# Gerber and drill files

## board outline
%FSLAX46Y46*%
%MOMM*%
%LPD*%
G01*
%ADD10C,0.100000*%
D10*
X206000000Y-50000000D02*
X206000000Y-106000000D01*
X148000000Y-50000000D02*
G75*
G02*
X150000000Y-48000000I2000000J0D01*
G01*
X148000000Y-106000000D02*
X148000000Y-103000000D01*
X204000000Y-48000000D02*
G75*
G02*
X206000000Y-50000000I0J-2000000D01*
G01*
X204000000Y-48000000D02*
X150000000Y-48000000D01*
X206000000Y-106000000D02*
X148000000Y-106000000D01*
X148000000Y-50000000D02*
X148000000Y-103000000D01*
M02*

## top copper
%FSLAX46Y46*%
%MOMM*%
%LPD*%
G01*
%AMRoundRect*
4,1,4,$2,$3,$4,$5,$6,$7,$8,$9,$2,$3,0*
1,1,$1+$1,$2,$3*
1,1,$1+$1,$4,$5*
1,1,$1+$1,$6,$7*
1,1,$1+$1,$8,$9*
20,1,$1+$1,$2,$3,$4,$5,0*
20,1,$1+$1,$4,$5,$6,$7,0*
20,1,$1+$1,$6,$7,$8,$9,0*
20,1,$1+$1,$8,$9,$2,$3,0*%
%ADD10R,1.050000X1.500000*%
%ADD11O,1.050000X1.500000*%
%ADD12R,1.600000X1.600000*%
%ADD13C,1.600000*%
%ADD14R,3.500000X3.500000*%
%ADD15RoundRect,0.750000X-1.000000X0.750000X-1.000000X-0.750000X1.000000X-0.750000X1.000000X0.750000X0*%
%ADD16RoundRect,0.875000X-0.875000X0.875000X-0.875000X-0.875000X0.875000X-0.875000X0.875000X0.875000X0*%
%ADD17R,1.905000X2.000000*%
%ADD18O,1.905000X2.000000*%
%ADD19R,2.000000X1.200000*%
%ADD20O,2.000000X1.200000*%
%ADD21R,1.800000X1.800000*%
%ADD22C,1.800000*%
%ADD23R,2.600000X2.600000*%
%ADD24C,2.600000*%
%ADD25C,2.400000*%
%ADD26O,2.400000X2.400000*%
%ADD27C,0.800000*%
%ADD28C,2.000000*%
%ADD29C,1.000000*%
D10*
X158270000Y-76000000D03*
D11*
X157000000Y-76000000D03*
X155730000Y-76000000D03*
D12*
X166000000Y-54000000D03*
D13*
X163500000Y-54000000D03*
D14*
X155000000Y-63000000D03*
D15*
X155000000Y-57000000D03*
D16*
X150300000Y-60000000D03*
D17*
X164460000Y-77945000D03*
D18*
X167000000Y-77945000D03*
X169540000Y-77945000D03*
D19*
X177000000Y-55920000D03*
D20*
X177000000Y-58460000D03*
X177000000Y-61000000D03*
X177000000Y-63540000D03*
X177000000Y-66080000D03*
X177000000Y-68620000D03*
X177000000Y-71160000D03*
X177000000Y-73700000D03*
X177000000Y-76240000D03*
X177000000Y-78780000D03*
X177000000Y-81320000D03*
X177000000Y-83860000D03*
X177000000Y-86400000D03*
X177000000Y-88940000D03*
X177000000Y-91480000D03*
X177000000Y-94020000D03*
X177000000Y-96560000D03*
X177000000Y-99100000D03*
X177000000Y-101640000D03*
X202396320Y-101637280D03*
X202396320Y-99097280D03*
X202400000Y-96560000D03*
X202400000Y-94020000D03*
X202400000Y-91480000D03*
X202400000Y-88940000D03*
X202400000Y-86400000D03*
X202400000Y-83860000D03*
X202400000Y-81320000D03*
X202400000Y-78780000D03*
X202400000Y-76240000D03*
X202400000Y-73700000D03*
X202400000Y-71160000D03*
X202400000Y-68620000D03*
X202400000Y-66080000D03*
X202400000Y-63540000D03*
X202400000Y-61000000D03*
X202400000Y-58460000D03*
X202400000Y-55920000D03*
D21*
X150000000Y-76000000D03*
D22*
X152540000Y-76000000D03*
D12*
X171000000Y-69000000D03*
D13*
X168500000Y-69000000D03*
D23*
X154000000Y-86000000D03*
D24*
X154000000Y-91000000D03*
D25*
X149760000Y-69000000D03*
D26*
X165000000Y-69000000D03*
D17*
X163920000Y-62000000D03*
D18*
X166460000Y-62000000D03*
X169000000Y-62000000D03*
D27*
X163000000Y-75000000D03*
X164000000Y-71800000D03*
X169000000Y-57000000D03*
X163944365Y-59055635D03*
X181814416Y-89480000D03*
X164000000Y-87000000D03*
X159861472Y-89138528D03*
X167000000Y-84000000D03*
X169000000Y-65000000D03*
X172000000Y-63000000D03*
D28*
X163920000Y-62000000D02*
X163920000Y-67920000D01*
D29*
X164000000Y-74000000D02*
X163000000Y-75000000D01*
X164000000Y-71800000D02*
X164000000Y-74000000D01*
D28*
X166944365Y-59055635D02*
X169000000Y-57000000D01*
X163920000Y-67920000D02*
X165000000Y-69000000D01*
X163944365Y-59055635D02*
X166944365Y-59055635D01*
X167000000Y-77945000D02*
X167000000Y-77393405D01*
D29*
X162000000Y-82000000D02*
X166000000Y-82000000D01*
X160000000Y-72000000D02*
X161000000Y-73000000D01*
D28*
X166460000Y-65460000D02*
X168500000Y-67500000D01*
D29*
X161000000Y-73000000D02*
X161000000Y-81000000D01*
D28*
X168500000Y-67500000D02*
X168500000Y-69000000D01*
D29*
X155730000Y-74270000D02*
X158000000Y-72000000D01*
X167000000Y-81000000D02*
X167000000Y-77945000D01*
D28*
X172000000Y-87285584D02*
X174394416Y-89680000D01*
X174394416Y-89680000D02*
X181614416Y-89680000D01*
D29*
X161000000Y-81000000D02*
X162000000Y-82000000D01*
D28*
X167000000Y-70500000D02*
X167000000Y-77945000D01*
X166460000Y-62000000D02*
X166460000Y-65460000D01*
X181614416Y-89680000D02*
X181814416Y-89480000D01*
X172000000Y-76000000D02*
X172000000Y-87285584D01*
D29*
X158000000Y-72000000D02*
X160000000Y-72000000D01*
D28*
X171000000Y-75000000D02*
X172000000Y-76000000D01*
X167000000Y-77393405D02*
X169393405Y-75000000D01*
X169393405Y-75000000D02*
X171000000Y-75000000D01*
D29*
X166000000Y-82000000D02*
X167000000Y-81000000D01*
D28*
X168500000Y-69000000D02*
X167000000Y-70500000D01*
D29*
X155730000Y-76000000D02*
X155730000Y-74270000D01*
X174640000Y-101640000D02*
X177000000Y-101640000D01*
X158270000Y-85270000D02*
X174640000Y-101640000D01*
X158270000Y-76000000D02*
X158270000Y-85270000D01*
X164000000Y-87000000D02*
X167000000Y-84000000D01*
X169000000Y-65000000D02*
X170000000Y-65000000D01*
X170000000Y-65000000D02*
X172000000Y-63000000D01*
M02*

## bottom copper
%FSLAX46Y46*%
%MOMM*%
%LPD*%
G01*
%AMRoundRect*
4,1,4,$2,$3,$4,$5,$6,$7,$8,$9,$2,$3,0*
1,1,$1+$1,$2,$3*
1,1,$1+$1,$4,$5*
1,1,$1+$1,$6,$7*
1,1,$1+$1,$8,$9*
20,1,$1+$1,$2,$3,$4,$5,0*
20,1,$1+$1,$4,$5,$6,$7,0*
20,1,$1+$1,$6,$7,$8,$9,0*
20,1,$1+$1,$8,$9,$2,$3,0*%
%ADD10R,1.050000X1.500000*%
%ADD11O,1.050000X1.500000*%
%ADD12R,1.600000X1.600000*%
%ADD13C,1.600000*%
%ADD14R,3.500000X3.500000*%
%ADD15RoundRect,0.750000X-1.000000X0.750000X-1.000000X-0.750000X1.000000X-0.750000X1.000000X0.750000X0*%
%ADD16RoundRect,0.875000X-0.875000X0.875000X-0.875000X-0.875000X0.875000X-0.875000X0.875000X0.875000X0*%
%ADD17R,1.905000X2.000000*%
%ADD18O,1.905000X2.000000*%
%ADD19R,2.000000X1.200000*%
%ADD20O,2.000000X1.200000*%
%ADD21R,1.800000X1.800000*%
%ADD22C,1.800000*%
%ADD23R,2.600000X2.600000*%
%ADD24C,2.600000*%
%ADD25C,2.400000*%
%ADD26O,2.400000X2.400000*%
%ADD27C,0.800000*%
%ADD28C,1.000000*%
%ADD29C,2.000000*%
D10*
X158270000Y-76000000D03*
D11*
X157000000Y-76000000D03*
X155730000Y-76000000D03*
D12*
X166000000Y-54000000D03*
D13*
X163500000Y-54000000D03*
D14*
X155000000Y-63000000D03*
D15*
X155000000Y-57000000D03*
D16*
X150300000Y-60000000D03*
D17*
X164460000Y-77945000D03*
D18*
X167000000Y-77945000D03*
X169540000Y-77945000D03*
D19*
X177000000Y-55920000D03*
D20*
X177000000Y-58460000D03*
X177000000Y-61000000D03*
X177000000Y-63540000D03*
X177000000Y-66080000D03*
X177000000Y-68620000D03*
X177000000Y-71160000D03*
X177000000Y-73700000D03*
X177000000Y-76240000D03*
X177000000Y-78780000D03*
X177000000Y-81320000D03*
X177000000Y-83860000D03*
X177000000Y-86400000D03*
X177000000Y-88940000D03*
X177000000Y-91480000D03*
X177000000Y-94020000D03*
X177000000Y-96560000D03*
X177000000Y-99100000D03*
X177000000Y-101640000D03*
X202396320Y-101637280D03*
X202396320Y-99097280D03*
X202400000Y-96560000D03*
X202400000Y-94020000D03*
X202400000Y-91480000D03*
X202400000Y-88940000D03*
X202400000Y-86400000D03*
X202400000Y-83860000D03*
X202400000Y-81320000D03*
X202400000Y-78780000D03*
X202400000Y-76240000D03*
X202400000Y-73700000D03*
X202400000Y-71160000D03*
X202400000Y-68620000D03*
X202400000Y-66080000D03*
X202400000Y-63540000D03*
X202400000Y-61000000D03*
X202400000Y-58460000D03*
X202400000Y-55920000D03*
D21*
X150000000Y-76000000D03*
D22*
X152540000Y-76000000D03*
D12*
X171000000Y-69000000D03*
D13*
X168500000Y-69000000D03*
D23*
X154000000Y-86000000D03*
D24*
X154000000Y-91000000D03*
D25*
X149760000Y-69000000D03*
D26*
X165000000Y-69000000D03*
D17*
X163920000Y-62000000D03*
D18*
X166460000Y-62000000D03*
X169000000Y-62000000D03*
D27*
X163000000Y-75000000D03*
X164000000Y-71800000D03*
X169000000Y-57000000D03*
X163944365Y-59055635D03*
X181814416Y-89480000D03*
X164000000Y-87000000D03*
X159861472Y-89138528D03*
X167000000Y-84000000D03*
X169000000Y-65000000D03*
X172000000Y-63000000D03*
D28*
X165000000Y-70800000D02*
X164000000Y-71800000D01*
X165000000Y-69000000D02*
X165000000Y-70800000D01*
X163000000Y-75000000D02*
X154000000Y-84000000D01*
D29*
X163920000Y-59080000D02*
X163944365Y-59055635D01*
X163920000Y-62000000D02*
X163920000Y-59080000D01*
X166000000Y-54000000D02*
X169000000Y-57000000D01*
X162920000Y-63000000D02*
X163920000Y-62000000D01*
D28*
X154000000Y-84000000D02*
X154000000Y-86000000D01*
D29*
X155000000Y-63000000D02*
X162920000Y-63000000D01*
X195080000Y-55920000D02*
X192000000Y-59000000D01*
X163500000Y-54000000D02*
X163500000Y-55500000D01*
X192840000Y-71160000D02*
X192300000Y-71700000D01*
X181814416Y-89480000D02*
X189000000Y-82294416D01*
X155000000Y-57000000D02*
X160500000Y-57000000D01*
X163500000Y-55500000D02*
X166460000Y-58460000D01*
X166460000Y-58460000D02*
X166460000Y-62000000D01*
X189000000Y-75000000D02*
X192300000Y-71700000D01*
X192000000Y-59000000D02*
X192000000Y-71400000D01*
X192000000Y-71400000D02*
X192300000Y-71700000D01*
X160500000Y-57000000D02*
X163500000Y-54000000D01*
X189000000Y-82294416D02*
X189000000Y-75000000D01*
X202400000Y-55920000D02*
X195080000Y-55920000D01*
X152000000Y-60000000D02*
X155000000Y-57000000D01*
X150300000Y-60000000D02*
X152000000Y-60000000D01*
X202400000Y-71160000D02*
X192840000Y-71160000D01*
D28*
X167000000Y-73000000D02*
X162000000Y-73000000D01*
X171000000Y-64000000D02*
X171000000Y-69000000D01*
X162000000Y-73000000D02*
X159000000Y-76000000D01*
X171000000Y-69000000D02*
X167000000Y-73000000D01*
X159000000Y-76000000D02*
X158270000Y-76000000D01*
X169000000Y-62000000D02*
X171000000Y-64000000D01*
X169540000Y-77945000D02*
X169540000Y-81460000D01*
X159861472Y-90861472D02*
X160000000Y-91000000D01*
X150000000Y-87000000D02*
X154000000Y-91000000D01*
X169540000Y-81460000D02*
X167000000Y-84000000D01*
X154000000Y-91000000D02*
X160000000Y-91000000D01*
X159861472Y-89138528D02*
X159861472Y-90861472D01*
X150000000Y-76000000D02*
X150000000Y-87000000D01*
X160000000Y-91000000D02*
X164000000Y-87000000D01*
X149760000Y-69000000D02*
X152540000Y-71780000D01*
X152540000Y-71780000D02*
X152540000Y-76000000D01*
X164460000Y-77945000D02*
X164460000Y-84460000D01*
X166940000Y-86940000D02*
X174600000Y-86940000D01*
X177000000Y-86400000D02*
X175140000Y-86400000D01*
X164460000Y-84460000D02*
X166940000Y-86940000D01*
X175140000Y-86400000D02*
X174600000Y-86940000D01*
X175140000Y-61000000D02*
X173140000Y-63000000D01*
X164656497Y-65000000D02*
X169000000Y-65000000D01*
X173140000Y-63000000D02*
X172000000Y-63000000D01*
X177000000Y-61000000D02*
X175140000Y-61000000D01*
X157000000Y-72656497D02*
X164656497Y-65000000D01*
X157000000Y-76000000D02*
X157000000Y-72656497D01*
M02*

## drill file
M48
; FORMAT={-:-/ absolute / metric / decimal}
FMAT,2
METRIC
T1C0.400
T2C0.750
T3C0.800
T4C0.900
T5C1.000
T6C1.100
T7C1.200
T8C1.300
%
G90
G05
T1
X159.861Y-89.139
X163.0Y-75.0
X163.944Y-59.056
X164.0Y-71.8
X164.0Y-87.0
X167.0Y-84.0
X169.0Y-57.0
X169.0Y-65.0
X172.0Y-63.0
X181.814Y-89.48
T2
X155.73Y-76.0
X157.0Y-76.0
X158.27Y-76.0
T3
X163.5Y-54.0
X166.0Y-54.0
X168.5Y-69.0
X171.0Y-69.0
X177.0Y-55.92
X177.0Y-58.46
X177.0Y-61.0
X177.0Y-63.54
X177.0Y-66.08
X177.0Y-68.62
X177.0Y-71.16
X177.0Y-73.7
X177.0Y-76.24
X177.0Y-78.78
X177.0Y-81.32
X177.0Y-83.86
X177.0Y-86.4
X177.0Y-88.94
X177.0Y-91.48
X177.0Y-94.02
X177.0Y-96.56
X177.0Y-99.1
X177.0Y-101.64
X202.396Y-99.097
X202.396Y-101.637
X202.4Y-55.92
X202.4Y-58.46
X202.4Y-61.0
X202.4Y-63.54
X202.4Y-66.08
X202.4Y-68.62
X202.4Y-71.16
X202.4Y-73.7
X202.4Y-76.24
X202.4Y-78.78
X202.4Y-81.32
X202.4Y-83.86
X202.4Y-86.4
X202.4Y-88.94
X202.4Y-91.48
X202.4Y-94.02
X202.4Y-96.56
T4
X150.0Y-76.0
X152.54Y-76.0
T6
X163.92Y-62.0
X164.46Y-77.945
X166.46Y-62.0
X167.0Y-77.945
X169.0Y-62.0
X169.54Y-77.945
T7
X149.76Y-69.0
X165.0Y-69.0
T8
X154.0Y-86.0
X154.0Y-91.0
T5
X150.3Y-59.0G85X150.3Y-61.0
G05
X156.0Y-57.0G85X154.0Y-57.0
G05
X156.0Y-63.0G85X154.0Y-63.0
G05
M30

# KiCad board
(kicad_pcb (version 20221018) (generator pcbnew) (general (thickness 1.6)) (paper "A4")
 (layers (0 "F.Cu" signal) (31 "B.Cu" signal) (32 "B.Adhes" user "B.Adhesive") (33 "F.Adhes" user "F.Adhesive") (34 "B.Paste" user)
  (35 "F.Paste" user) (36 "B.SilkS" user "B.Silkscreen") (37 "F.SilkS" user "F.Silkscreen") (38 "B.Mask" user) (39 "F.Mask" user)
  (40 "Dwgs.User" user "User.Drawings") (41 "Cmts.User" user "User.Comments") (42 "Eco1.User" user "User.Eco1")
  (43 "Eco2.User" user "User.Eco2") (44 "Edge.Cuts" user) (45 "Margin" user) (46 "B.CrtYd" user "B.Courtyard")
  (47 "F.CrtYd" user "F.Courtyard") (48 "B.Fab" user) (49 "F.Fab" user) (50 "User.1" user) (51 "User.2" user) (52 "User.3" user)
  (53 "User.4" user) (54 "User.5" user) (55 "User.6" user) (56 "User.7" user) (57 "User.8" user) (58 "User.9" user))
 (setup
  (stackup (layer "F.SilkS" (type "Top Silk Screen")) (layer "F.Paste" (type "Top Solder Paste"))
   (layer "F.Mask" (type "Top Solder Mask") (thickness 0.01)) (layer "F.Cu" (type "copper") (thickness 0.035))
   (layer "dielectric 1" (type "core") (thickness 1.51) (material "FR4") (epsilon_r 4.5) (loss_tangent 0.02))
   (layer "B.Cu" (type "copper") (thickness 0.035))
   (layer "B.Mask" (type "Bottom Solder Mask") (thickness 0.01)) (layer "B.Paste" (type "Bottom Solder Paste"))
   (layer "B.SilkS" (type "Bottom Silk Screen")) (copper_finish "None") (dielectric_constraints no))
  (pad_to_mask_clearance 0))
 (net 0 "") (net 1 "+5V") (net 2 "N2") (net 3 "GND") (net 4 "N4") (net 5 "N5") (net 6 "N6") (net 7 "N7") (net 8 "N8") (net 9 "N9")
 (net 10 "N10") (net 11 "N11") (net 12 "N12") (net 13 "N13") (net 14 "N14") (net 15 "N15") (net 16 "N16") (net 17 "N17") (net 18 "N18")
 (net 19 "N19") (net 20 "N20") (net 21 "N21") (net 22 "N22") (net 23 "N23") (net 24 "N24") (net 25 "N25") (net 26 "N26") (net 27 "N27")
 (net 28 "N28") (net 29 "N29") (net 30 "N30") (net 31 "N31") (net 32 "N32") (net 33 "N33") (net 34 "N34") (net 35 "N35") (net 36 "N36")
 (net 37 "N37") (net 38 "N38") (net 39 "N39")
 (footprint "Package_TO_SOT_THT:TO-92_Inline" (layer "F.Cu") (at 158.27 76 180)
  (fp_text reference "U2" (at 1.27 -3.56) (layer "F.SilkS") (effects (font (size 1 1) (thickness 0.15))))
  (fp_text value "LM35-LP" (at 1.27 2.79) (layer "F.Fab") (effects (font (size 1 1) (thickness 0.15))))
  (pad "1" thru_hole rect (at 0 0 180) (size 1.05 1.5) (drill 0.75) (layers "*.Cu" "*.Mask") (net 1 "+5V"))
  (pad "2" thru_hole oval (at 1.27 0 180) (size 1.05 1.5) (drill 0.75) (layers "*.Cu" "*.Mask") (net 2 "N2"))
  (pad "3" thru_hole oval (at 2.54 0 180) (size 1.05 1.5) (drill 0.75) (layers "*.Cu" "*.Mask") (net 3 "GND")))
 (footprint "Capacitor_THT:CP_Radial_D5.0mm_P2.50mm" (layer "F.Cu") (at 166 54 180)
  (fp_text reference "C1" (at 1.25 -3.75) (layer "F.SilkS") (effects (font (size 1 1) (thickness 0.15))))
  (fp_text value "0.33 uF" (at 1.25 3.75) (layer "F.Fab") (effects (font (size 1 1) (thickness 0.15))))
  (pad "1" thru_hole rect (at 0 0 180) (size 1.6 1.6) (drill 0.8) (layers "*.Cu" "*.Mask") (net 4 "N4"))
  (pad "2" thru_hole circle (at 2.5 0 180) (size 1.6 1.6) (drill 0.8) (layers "*.Cu" "*.Mask") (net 3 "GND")))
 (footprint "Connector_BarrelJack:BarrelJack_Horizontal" (layer "F.Cu") (at 155 63 -90)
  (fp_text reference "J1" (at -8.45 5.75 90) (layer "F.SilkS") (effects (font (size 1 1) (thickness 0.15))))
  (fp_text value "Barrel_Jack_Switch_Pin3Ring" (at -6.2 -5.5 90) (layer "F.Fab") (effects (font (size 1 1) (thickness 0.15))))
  (pad "1" thru_hole rect (at 0 0 270) (size 3.5 3.5) (drill oval 1 3) (layers "*.Cu" "*.Mask") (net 4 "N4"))
  (pad "2" thru_hole roundrect (at -6 0 270) (size 3 3.5) (drill oval 1 3) (layers "*.Cu" "*.Mask") (roundrect_rratio 0.25) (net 3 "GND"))
  (pad "3" thru_hole roundrect (at -3 4.7 270) (size 3.5 3.5) (drill oval 3 1) (layers "*.Cu" "*.Mask") (roundrect_rratio 0.25)
   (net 3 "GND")))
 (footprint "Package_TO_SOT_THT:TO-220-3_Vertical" (layer "F.Cu") (at 164.46 77.945)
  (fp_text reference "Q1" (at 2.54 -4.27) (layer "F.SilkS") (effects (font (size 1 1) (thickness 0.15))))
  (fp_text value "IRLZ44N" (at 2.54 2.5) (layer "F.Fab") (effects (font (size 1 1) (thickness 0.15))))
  (pad "1" thru_hole rect (at 0 0) (size 1.905 2) (drill 1.1) (layers "*.Cu" "*.Mask") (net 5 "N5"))
  (pad "2" thru_hole oval (at 2.54 0) (size 1.905 2) (drill 1.1) (layers "*.Cu" "*.Mask") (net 3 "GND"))
  (pad "3" thru_hole oval (at 5.08 0) (size 1.905 2) (drill 1.1) (layers "*.Cu" "*.Mask") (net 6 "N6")))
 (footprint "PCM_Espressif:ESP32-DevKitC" (layer "F.Cu") (at 177 55.92)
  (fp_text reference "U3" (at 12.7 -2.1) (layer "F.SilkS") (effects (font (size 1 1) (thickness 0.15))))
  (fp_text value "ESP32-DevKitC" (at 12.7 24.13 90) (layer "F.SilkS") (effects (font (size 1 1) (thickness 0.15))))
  (pad "1" thru_hole rect (at 0 0 270) (size 1.2 2) (drill 0.8) (layers "*.Cu" "*.Mask") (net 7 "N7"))
  (pad "2" thru_hole oval (at 0 2.54 270) (size 1.2 2) (drill 0.8) (layers "*.Cu" "*.Mask") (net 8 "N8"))
  (pad "3" thru_hole oval (at 0 5.08 270) (size 1.2 2) (drill 0.8) (layers "*.Cu" "*.Mask") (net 2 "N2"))
  (pad "4" thru_hole oval (at 0 7.62 270) (size 1.2 2) (drill 0.8) (layers "*.Cu" "*.Mask") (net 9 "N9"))
  (pad "5" thru_hole oval (at 0 10.16 270) (size 1.2 2) (drill 0.8) (layers "*.Cu" "*.Mask") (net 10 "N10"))
  (pad "6" thru_hole oval (at 0 12.7 270) (size 1.2 2) (drill 0.8) (layers "*.Cu" "*.Mask") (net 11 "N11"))
  (pad "7" thru_hole oval (at 0 15.24 270) (size 1.2 2) (drill 0.8) (layers "*.Cu" "*.Mask") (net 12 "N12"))
  (pad "8" thru_hole oval (at 0 17.78 270) (size 1.2 2) (drill 0.8) (layers "*.Cu" "*.Mask") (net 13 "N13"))
  (pad "9" thru_hole oval (at 0 20.32 270) (size 1.2 2) (drill 0.8) (layers "*.Cu" "*.Mask") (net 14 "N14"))
  (pad "10" thru_hole oval (at 0 22.86 270) (size 1.2 2) (drill 0.8) (layers "*.Cu" "*.Mask") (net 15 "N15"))
  (pad "11" thru_hole oval (at 0 25.4 270) (size 1.2 2) (drill 0.8) (layers "*.Cu" "*.Mask") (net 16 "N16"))
  (pad "12" thru_hole oval (at 0 27.94 270) (size 1.2 2) (drill 0.8) (layers "*.Cu" "*.Mask") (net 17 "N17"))
  (pad "13" thru_hole oval (at 0 30.48 270) (size 1.2 2) (drill 0.8) (layers "*.Cu" "*.Mask") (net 5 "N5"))
  (pad "14" thru_hole oval (at 0 33.02 270) (size 1.2 2) (drill 0.8) (layers "*.Cu" "*.Mask") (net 3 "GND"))
  (pad "15" thru_hole oval (at 0 35.56 270) (size 1.2 2) (drill 0.8) (layers "*.Cu" "*.Mask") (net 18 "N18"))
  (pad "16" thru_hole oval (at 0 38.1 270) (size 1.2 2) (drill 0.8) (layers "*.Cu" "*.Mask") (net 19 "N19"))
  (pad "17" thru_hole oval (at 0 40.64 270) (size 1.2 2) (drill 0.8) (layers "*.Cu" "*.Mask") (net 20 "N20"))
  (pad "18" thru_hole oval (at 0 43.18 270) (size 1.2 2) (drill 0.8) (layers "*.Cu" "*.Mask") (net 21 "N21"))
  (pad "19" thru_hole oval (at 0 45.72 270) (size 1.2 2) (drill 0.8) (layers "*.Cu" "*.Mask") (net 1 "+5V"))
  (pad "20" thru_hole oval (at 25.39632 45.71728 270) (size 1.2 2) (drill 0.8) (layers "*.Cu" "*.Mask") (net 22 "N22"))
  (pad "21" thru_hole oval (at 25.39632 43.17728 270) (size 1.2 2) (drill 0.8) (layers "*.Cu" "*.Mask") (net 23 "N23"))
  (pad "22" thru_hole oval (at 25.4 40.64 270) (size 1.2 2) (drill 0.8) (layers "*.Cu" "*.Mask") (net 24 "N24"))
  (pad "23" thru_hole oval (at 25.4 38.1 270) (size 1.2 2) (drill 0.8) (layers "*.Cu" "*.Mask") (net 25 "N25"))
  (pad "24" thru_hole oval (at 25.4 35.56 270) (size 1.2 2) (drill 0.8) (layers "*.Cu" "*.Mask") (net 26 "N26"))
  (pad "25" thru_hole oval (at 25.4 33.02 270) (size 1.2 2) (drill 0.8) (layers "*.Cu" "*.Mask") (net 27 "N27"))
  (pad "26" thru_hole oval (at 25.4 30.48 270) (size 1.2 2) (drill 0.8) (layers "*.Cu" "*.Mask") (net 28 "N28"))
  (pad "27" thru_hole oval (at 25.4 27.94 270) (size 1.2 2) (drill 0.8) (layers "*.Cu" "*.Mask") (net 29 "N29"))
  (pad "28" thru_hole oval (at 25.4 25.4 270) (size 1.2 2) (drill 0.8) (layers "*.Cu" "*.Mask") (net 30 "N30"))
  (pad "29" thru_hole oval (at 25.4 22.86 270) (size 1.2 2) (drill 0.8) (layers "*.Cu" "*.Mask") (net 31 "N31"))
  (pad "30" thru_hole oval (at 25.4 20.32 270) (size 1.2 2) (drill 0.8) (layers "*.Cu" "*.Mask") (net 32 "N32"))
  (pad "31" thru_hole oval (at 25.4 17.78 270) (size 1.2 2) (drill 0.8) (layers "*.Cu" "*.Mask") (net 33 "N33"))
  (pad "32" thru_hole oval (at 25.4 15.24 270) (size 1.2 2) (drill 0.8) (layers "*.Cu" "*.Mask") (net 3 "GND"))
  (pad "33" thru_hole oval (at 25.4 12.7 270) (size 1.2 2) (drill 0.8) (layers "*.Cu" "*.Mask") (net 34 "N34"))
  (pad "34" thru_hole oval (at 25.4 10.16 270) (size 1.2 2) (drill 0.8) (layers "*.Cu" "*.Mask") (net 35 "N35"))
  (pad "35" thru_hole oval (at 25.4 7.62 270) (size 1.2 2) (drill 0.8) (layers "*.Cu" "*.Mask") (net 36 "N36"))
  (pad "36" thru_hole oval (at 25.4 5.08 270) (size 1.2 2) (drill 0.8) (layers "*.Cu" "*.Mask") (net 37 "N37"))
  (pad "37" thru_hole oval (at 25.4 2.54 270) (size 1.2 2) (drill 0.8) (layers "*.Cu" "*.Mask") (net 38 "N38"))
  (pad "38" thru_hole oval (at 25.4 0 270) (size 1.2 2) (drill 0.8) (layers "*.Cu" "*.Mask") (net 3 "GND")))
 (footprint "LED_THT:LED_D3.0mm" (layer "F.Cu") (at 150 76)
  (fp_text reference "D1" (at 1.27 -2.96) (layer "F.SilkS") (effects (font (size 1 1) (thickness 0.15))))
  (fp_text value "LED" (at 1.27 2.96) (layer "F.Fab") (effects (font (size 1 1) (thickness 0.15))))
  (pad "1" thru_hole rect (at 0 0) (size 1.8 1.8) (drill 0.9) (layers "*.Cu" "*.Mask") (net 6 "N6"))
  (pad "2" thru_hole circle (at 2.54 0) (size 1.8 1.8) (drill 0.9) (layers "*.Cu" "*.Mask") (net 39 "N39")))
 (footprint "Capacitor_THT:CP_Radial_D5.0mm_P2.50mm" (layer "F.Cu") (at 171 69 180)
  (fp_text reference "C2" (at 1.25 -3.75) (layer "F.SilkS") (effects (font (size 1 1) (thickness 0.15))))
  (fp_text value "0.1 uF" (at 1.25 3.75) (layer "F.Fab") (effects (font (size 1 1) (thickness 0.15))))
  (pad "1" thru_hole rect (at 0 0 180) (size 1.6 1.6) (drill 0.8) (layers "*.Cu" "*.Mask") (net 1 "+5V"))
  (pad "2" thru_hole circle (at 2.5 0 180) (size 1.6 1.6) (drill 0.8) (layers "*.Cu" "*.Mask") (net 3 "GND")))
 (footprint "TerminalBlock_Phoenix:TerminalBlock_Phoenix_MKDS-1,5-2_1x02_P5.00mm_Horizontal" (layer "F.Cu") (at 154 86 -90)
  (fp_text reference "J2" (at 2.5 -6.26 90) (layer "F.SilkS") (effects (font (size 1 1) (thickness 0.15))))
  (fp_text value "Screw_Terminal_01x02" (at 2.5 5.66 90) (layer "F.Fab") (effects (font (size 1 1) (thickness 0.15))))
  (pad "1" thru_hole rect (at 0 0 270) (size 2.6 2.6) (drill 1.3) (layers "*.Cu" "*.Mask") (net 4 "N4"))
  (pad "2" thru_hole circle (at 5 0 270) (size 2.6 2.6) (drill 1.3) (layers "*.Cu" "*.Mask") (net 6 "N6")))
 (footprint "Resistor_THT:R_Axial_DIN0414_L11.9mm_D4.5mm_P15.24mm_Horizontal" (layer "F.Cu") (at 149.76 69)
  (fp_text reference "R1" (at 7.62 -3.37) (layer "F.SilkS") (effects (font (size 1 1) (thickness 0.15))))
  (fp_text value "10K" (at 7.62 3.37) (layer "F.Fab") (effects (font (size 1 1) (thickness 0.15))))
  (pad "1" thru_hole circle (at 0 0) (size 2.4 2.4) (drill 1.2) (layers "*.Cu" "*.Mask") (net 39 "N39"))
  (pad "2" thru_hole oval (at 15.24 0) (size 2.4 2.4) (drill 1.2) (layers "*.Cu" "*.Mask") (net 4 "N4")))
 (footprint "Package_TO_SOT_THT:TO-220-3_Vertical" (layer "F.Cu") (at 163.92 62)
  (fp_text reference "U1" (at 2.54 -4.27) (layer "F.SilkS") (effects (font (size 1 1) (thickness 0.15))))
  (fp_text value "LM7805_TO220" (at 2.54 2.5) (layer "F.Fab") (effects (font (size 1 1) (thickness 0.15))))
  (pad "1" thru_hole rect (at 0 0) (size 1.905 2) (drill 1.1) (layers "*.Cu" "*.Mask") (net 4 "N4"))
  (pad "2" thru_hole oval (at 2.54 0) (size 1.905 2) (drill 1.1) (layers "*.Cu" "*.Mask") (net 3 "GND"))
  (pad "3" thru_hole oval (at 5.08 0) (size 1.905 2) (drill 1.1) (layers "*.Cu" "*.Mask") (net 1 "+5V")))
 (gr_line (start 206 50) (end 206 106) (stroke (width 0.1) (type default)) (layer "Edge.Cuts"))
 (gr_arc (start 148 50) (mid 148.585786 48.585786) (end 150 48) (stroke (width 0.1) (type default)) (layer "Edge.Cuts"))
 (gr_line (start 148 106) (end 148 103) (stroke (width 0.1) (type default)) (layer "Edge.Cuts"))
 (gr_arc (start 204 48) (mid 205.414214 48.585786) (end 206 50) (stroke (width 0.1) (type default)) (layer "Edge.Cuts"))
 (gr_line (start 204 48) (end 150 48) (stroke (width 0.1) (type default)) (layer "Edge.Cuts"))
 (gr_line (start 206 106) (end 148 106) (stroke (width 0.1) (type default)) (layer "Edge.Cuts"))
 (gr_line (start 148 50) (end 148 103) (stroke (width 0.1) (type default)) (layer "Edge.Cuts"))
 (segment (start 163.92 62) (end 163.92 67.92) (width 2) (layer "F.Cu") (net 4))
 (segment (start 164 74) (end 163 75) (width 1) (layer "F.Cu") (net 4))
 (segment (start 164 71.8) (end 164 74) (width 1) (layer "F.Cu") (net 4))
 (segment (start 166.944365 59.055635) (end 169 57) (width 2) (layer "F.Cu") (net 4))
 (segment (start 163.92 67.92) (end 165 69) (width 2) (layer "F.Cu") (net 4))
 (segment (start 163.944365 59.055635) (end 166.944365 59.055635) (width 2) (layer "F.Cu") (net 4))
 (via (at 163 75) (size 0.8) (drill 0.4) (layers "F.Cu" "B.Cu") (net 4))
 (via (at 164 71.8) (size 0.8) (drill 0.4) (layers "F.Cu" "B.Cu") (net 4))
 (via (at 169 57) (size 0.8) (drill 0.4) (layers "F.Cu" "B.Cu") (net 4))
 (via (at 163.944365 59.055635) (size 0.8) (drill 0.4) (layers "F.Cu" "B.Cu") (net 4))
 (segment (start 165 70.8) (end 164 71.8) (width 1) (layer "B.Cu") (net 4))
 (segment (start 165 69) (end 165 70.8) (width 1) (layer "B.Cu") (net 4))
 (segment (start 163 75) (end 154 84) (width 1) (layer "B.Cu") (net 4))
 (segment (start 163.92 59.08) (end 163.944365 59.055635) (width 2) (layer "B.Cu") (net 4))
 (segment (start 163.92 62) (end 163.92 59.08) (width 2) (layer "B.Cu") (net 4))
 (segment (start 166 54) (end 169 57) (width 2) (layer "B.Cu") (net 4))
 (segment (start 162.92 63) (end 163.92 62) (width 2) (layer "B.Cu") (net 4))
 (segment (start 154 84) (end 154 86) (width 1) (layer "B.Cu") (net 4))
 (segment (start 155 63) (end 162.92 63) (width 2) (layer "B.Cu") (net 4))
 (segment (start 167 77.945) (end 167 77.393405) (width 2) (layer "F.Cu") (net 3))
 (segment (start 162 82) (end 166 82) (width 1) (layer "F.Cu") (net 3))
 (segment (start 160 72) (end 161 73) (width 1) (layer "F.Cu") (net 3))
 (segment (start 166.46 65.46) (end 168.5 67.5) (width 2) (layer "F.Cu") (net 3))
 (segment (start 161 73) (end 161 81) (width 1) (layer "F.Cu") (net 3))
 (segment (start 168.5 67.5) (end 168.5 69) (width 2) (layer "F.Cu") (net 3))
 (segment (start 155.73 74.27) (end 158 72) (width 1) (layer "F.Cu") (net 3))
 (segment (start 167 81) (end 167 77.945) (width 1) (layer "F.Cu") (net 3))
 (segment (start 172 87.285584) (end 174.394416 89.68) (width 2) (layer "F.Cu") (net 3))
 (segment (start 174.394416 89.68) (end 181.614416 89.68) (width 2) (layer "F.Cu") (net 3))
 (segment (start 161 81) (end 162 82) (width 1) (layer "F.Cu") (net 3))
 (segment (start 167 70.5) (end 167 77.945) (width 2) (layer "F.Cu") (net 3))
 (segment (start 166.46 62) (end 166.46 65.46) (width 2) (layer "F.Cu") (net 3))
 (segment (start 181.614416 89.68) (end 181.814416 89.48) (width 2) (layer "F.Cu") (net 3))
 (segment (start 172 76) (end 172 87.285584) (width 2) (layer "F.Cu") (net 3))
 (segment (start 158 72) (end 160 72) (width 1) (layer "F.Cu") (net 3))
 (segment (start 171 75) (end 172 76) (width 2) (layer "F.Cu") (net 3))
 (segment (start 167 77.393405) (end 169.393405 75) (width 2) (layer "F.Cu") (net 3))
 (segment (start 169.393405 75) (end 171 75) (width 2) (layer "F.Cu") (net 3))
 (segment (start 166 82) (end 167 81) (width 1) (layer "F.Cu") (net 3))
 (segment (start 168.5 69) (end 167 70.5) (width 2) (layer "F.Cu") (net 3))
 (segment (start 155.73 76) (end 155.73 74.27) (width 1) (layer "F.Cu") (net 3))
 (via (at 181.814416 89.48) (size 0.8) (drill 0.4) (layers "F.Cu" "B.Cu") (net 3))
 (segment (start 195.08 55.92) (end 192 59) (width 2) (layer "B.Cu") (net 3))
 (segment (start 163.5 54) (end 163.5 55.5) (width 2) (layer "B.Cu") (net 3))
 (segment (start 192.84 71.16) (end 192.3 71.7) (width 2) (layer "B.Cu") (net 3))
 (segment (start 181.814416 89.48) (end 189 82.294416) (width 2) (layer "B.Cu") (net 3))
 (segment (start 155 57) (end 160.5 57) (width 2) (layer "B.Cu") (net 3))
 (segment (start 163.5 55.5) (end 166.46 58.46) (width 2) (layer "B.Cu") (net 3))
 (segment (start 166.46 58.46) (end 166.46 62) (width 2) (layer "B.Cu") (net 3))
 (segment (start 189 75) (end 192.3 71.7) (width 2) (layer "B.Cu") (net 3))
 (segment (start 192 59) (end 192 71.4) (width 2) (layer "B.Cu") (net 3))
 (segment (start 192 71.4) (end 192.3 71.7) (width 2) (layer "B.Cu") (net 3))
 (segment (start 160.5 57) (end 163.5 54) (width 2) (layer "B.Cu") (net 3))
 (segment (start 189 82.294416) (end 189 75) (width 2) (layer "B.Cu") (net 3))
 (segment (start 202.4 55.92) (end 195.08 55.92) (width 2) (layer "B.Cu") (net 3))
 (segment (start 152 60) (end 155 57) (width 2) (layer "B.Cu") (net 3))
 (segment (start 150.3 60) (end 152 60) (width 2) (layer "B.Cu") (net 3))
 (segment (start 202.4 71.16) (end 192.84 71.16) (width 2) (layer "B.Cu") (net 3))
 (segment (start 174.64 101.64) (end 177 101.64) (width 1) (layer "F.Cu") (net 1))
 (segment (start 158.27 85.27) (end 174.64 101.64) (width 1) (layer "F.Cu") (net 1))
 (segment (start 158.27 76) (end 158.27 85.27) (width 1) (layer "F.Cu") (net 1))
 (segment (start 167 73) (end 162 73) (width 1) (layer "B.Cu") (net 1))
 (segment (start 171 64) (end 171 69) (width 1) (layer "B.Cu") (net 1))
 (segment (start 162 73) (end 159 76) (width 1) (layer "B.Cu") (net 1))
 (segment (start 171 69) (end 167 73) (width 1) (layer "B.Cu") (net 1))
 (segment (start 159 76) (end 158.27 76) (width 1) (layer "B.Cu") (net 1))
 (segment (start 169 62) (end 171 64) (width 1) (layer "B.Cu") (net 1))
 (segment (start 164 87) (end 167 84) (width 1) (layer "F.Cu") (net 6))
 (via (at 164 87) (size 0.8) (drill 0.4) (layers "F.Cu" "B.Cu") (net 6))
 (via (at 159.861472 89.138528) (size 0.8) (drill 0.4) (layers "F.Cu" "B.Cu") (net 6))
 (via (at 167 84) (size 0.8) (drill 0.4) (layers "F.Cu" "B.Cu") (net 6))
 (segment (start 169.54 77.945) (end 169.54 81.46) (width 1) (layer "B.Cu") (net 6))
 (segment (start 159.861472 90.861472) (end 160 91) (width 1) (layer "B.Cu") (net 6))
 (segment (start 150 87) (end 154 91) (width 1) (layer "B.Cu") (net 6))
 (segment (start 169.54 81.46) (end 167 84) (width 1) (layer "B.Cu") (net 6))
 (segment (start 154 91) (end 160 91) (width 1) (layer "B.Cu") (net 6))
 (segment (start 159.861472 89.138528) (end 159.861472 90.861472) (width 1) (layer "B.Cu") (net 6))
 (segment (start 150 76) (end 150 87) (width 1) (layer "B.Cu") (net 6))
 (segment (start 160 91) (end 164 87) (width 1) (layer "B.Cu") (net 6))
 (segment (start 149.76 69) (end 152.54 71.78) (width 1) (layer "B.Cu") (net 39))
 (segment (start 152.54 71.78) (end 152.54 76) (width 1) (layer "B.Cu") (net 39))
 (segment (start 164.46 77.945) (end 164.46 84.46) (width 1) (layer "B.Cu") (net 5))
 (segment (start 166.94 86.94) (end 174.6 86.94) (width 1) (layer "B.Cu") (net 5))
 (segment (start 177 86.4) (end 175.14 86.4) (width 1) (layer "B.Cu") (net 5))
 (segment (start 164.46 84.46) (end 166.94 86.94) (width 1) (layer "B.Cu") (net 5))
 (segment (start 175.14 86.4) (end 174.6 86.94) (width 1) (layer "B.Cu") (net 5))
 (segment (start 169 65) (end 170 65) (width 1) (layer "F.Cu") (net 2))
 (segment (start 170 65) (end 172 63) (width 1) (layer "F.Cu") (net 2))
 (via (at 169 65) (size 0.8) (drill 0.4) (layers "F.Cu" "B.Cu") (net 2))
 (via (at 172 63) (size 0.8) (drill 0.4) (layers "F.Cu" "B.Cu") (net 2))
 (segment (start 175.14 61) (end 173.14 63) (width 1) (layer "B.Cu") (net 2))
 (segment (start 164.656497 65) (end 169 65) (width 1) (layer "B.Cu") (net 2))
 (segment (start 173.14 63) (end 172 63) (width 1) (layer "B.Cu") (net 2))
 (segment (start 177 61) (end 175.14 61) (width 1) (layer "B.Cu") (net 2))
 (segment (start 157 72.656497) (end 164.656497 65) (width 1) (layer "B.Cu") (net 2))
 (segment (start 157 76) (end 157 72.656497) (width 1) (layer "B.Cu") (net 2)))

